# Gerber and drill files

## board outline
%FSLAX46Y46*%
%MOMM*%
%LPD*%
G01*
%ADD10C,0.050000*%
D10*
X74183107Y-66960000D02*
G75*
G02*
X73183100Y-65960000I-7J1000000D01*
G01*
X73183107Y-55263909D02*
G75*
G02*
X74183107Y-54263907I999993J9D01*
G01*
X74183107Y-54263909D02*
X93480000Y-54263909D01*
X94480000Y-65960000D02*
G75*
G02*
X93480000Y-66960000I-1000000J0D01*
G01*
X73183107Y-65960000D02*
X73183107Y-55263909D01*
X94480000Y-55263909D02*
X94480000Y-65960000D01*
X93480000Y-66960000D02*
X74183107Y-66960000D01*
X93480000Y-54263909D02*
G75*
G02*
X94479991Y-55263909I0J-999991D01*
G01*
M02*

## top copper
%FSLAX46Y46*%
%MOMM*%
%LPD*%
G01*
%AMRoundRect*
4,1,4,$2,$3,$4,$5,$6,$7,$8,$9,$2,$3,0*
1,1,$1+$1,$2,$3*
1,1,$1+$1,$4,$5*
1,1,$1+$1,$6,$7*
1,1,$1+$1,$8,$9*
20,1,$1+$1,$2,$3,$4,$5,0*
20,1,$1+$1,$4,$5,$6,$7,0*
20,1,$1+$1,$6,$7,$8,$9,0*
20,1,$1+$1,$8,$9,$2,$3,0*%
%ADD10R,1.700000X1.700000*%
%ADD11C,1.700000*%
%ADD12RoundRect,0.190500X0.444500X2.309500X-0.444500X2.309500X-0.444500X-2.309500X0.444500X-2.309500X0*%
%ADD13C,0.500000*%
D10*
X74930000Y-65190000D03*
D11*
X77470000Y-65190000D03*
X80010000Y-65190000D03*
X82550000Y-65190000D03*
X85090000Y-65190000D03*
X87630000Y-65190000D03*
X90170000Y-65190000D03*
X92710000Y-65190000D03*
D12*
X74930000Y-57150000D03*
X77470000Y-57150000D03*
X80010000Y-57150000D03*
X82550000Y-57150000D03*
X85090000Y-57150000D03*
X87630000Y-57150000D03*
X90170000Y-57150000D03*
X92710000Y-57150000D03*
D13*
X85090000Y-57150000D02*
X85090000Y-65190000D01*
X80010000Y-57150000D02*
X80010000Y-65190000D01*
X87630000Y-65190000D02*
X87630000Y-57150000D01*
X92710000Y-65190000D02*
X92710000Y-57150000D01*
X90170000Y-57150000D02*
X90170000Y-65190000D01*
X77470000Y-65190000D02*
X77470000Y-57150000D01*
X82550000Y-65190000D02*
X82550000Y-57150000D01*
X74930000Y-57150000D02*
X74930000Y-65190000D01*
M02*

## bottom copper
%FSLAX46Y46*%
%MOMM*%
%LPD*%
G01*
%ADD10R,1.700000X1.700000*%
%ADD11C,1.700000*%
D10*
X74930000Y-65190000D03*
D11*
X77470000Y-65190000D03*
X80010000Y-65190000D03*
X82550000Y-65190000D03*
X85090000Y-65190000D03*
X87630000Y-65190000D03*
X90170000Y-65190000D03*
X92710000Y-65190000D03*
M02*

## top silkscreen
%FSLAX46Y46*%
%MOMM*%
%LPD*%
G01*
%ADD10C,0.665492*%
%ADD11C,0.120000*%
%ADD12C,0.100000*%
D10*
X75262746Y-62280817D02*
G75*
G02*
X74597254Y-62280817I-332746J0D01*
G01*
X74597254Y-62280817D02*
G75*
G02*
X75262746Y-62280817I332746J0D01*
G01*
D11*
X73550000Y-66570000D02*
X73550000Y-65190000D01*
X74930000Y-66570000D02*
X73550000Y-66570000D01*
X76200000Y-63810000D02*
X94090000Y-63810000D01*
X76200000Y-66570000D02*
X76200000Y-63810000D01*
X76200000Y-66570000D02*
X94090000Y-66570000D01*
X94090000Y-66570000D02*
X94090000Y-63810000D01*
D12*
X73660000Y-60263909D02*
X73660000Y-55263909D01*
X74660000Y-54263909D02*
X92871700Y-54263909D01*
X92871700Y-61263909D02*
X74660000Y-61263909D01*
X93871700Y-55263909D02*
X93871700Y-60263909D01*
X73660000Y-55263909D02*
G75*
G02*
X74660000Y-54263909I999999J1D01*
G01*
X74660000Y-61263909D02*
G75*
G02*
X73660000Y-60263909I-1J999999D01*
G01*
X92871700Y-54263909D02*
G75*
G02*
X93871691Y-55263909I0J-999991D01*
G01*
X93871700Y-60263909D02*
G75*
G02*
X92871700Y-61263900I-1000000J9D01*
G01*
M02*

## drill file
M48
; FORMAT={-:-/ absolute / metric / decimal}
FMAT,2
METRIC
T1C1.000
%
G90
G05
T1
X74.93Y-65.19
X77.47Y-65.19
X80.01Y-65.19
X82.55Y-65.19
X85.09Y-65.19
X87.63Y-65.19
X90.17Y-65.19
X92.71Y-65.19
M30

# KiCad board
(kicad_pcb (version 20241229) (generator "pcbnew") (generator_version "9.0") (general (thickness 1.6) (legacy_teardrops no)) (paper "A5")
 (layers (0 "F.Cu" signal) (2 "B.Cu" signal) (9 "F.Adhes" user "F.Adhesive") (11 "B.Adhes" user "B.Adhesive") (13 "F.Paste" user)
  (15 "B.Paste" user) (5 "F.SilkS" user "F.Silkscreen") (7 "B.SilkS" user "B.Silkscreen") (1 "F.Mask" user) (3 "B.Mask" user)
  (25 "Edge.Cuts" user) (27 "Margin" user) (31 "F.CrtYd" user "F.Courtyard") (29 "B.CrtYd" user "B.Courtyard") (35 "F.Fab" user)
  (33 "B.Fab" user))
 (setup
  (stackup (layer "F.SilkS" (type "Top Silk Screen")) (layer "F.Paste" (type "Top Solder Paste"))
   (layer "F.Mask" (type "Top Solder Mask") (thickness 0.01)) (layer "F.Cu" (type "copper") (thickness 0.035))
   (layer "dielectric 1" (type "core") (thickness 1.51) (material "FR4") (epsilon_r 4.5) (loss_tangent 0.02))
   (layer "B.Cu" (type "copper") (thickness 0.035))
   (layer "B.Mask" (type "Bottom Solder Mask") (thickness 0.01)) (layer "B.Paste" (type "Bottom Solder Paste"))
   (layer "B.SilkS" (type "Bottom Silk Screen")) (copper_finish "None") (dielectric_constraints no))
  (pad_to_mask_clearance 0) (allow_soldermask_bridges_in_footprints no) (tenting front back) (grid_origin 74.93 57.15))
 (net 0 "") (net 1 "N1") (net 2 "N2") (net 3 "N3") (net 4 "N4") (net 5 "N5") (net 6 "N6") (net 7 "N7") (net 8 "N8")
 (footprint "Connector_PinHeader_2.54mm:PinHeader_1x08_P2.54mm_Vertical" (layer "F.Cu") (at 74.93 65.19 90)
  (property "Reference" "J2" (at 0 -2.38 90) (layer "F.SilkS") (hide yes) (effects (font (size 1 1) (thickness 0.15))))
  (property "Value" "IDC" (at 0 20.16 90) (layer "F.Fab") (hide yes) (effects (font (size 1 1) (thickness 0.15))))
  (fp_line (start -1.38 -1.38) (end 0 -1.38) (stroke (width 0.12) (type solid)) (layer "F.SilkS"))
  (fp_line (start -1.38 0) (end -1.38 -1.38) (stroke (width 0.12) (type solid)) (layer "F.SilkS"))
  (fp_line (start 1.38 1.27) (end 1.38 19.16) (stroke (width 0.12) (type solid)) (layer "F.SilkS"))
  (fp_line (start -1.38 1.27) (end 1.38 1.27) (stroke (width 0.12) (type solid)) (layer "F.SilkS"))
  (fp_line (start -1.38 1.27) (end -1.38 19.16) (stroke (width 0.12) (type solid)) (layer "F.SilkS"))
  (fp_line (start -1.38 19.16) (end 1.38 19.16) (stroke (width 0.12) (type solid)) (layer "F.SilkS"))
  (pad "1" thru_hole rect (at 0 0 90) (size 1.7 1.7) (drill 1) (layers "*.Cu" "*.Mask") (remove_unused_layers no) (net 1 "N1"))
  (pad "2" thru_hole circle (at 0 2.54 90) (size 1.7 1.7) (drill 1) (layers "*.Cu" "*.Mask") (remove_unused_layers no) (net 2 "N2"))
  (pad "3" thru_hole circle (at 0 5.08 90) (size 1.7 1.7) (drill 1) (layers "*.Cu" "*.Mask") (remove_unused_layers no) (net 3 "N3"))
  (pad "4" thru_hole circle (at 0 7.62 90) (size 1.7 1.7) (drill 1) (layers "*.Cu" "*.Mask") (remove_unused_layers no) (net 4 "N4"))
  (pad "5" thru_hole circle (at 0 10.16 90) (size 1.7 1.7) (drill 1) (layers "*.Cu" "*.Mask") (remove_unused_layers no) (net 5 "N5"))
  (pad "6" thru_hole circle (at 0 12.7 90) (size 1.7 1.7) (drill 1) (layers "*.Cu" "*.Mask") (remove_unused_layers no) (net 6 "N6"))
  (pad "7" thru_hole circle (at 0 15.24 90) (size 1.7 1.7) (drill 1) (layers "*.Cu" "*.Mask") (remove_unused_layers no) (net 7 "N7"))
  (pad "8" thru_hole circle (at 0 17.78 90) (size 1.7 1.7) (drill 1) (layers "*.Cu" "*.Mask") (remove_unused_layers no) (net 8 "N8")))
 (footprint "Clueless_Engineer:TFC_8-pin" (layer "F.Cu") (at 83.82 57.15)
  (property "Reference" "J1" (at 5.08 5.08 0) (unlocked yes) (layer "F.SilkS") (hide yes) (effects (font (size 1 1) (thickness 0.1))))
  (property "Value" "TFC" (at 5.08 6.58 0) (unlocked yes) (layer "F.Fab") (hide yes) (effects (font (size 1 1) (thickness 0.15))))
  (fp_line (start -10.16 3.113909) (end -10.16 -1.886091) (stroke (width 0.1) (type default)) (layer "F.SilkS"))
  (fp_line (start -9.16 -2.886091) (end 9.0517 -2.886091) (stroke (width 0.1) (type default)) (layer "F.SilkS"))
  (fp_line (start 9.0517 4.113909) (end -9.16 4.113909) (stroke (width 0.1) (type default)) (layer "F.SilkS"))
  (fp_line (start 10.0517 -1.886091) (end 10.0517 3.113909) (stroke (width 0.1) (type default)) (layer "F.SilkS"))
  (fp_arc (start -10.16 -1.886091) (mid -9.867107 -2.593198) (end -9.16 -2.886091) (stroke (width 0.1) (type default)) (layer "F.SilkS"))
  (fp_arc (start -9.16 4.113909) (mid -9.867107 3.821016) (end -10.16 3.113909) (stroke (width 0.1) (type default)) (layer "F.SilkS"))
  (fp_arc (start 9.0517 -2.886091) (mid 9.758804 -2.593197) (end 10.0517 -1.886091) (stroke (width 0.1) (type default)) (layer "F.SilkS"))
  (fp_arc (start 10.0517 3.113909) (mid 9.758804 3.82101) (end 9.0517 4.113909) (stroke (width 0.1) (type default)) (layer "F.SilkS"))
  (pad "1" connect roundrect (at -8.89 0 180) (size 1.27 5) (layers "F.Cu" "F.Mask") (roundrect_rratio 0.15) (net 1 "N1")
   (thermal_bridge_angle 45))
  (pad "2" connect roundrect (at -6.35 0 180) (size 1.27 5) (layers "F.Cu" "F.Mask") (roundrect_rratio 0.15) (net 2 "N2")
   (thermal_bridge_angle 45))
  (pad "3" connect roundrect (at -3.81 0 180) (size 1.27 5) (layers "F.Cu" "F.Mask") (roundrect_rratio 0.15) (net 3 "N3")
   (thermal_bridge_angle 45))
  (pad "4" connect roundrect (at -1.27 0 180) (size 1.27 5) (layers "F.Cu" "F.Mask") (roundrect_rratio 0.15) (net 4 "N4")
   (thermal_bridge_angle 45))
  (pad "5" connect roundrect (at 1.27 0 180) (size 1.27 5) (layers "F.Cu" "F.Mask") (roundrect_rratio 0.15) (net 5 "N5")
   (thermal_bridge_angle 45))
  (pad "6" connect roundrect (at 3.81 0 180) (size 1.27 5) (layers "F.Cu" "F.Mask") (roundrect_rratio 0.15) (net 6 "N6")
   (thermal_bridge_angle 45))
  (pad "7" connect roundrect (at 6.35 0 180) (size 1.27 5) (layers "F.Cu" "F.Mask") (roundrect_rratio 0.15) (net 7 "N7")
   (thermal_bridge_angle 45))
  (pad "8" connect roundrect (at 8.89 0 180) (size 1.27 5) (layers "F.Cu" "F.Mask") (roundrect_rratio 0.15) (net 8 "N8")
   (thermal_bridge_angle 45)))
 (gr_circle (center 74.93 62.280817) (end 75.530484 62.415908) (stroke (width 0.1) (type solid)) (fill yes) (layer "F.SilkS"))
 (gr_arc (start 74.183107 66.96) (mid 73.475996 66.667109) (end 73.183107 65.96) (stroke (width 0.05) (type default)) (layer "Edge.Cuts"))
 (gr_arc (start 73.183107 55.263909) (mid 73.476 54.556802) (end 74.183107 54.263909) (stroke (width 0.05) (type default))
  (layer "Edge.Cuts"))
 (gr_line (start 74.183107 54.263909) (end 93.48 54.263909) (stroke (width 0.05) (type default)) (layer "Edge.Cuts"))
 (gr_arc (start 94.48 65.96) (mid 94.187107 66.667107) (end 93.48 66.96) (stroke (width 0.05) (type default)) (layer "Edge.Cuts"))
 (gr_line (start 73.183107 65.96) (end 73.183107 55.263909) (stroke (width 0.05) (type default)) (layer "Edge.Cuts"))
 (gr_line (start 94.48 55.263909) (end 94.48 65.96) (stroke (width 0.05) (type default)) (layer "Edge.Cuts"))
 (gr_line (start 93.48 66.96) (end 74.183107 66.96) (stroke (width 0.05) (type default)) (layer "Edge.Cuts"))
 (gr_arc (start 93.48 54.263909) (mid 94.187104 54.556803) (end 94.48 55.263909) (stroke (width 0.05) (type default)) (layer "Edge.Cuts"))
 (segment (start 85.09 57.15) (end 85.09 65.19) (width 0.5) (layer "F.Cu") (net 5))
 (segment (start 80.01 57.15) (end 80.01 65.19) (width 0.5) (layer "F.Cu") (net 3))
 (segment (start 87.63 65.19) (end 87.63 57.15) (width 0.5) (layer "F.Cu") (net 6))
 (segment (start 92.71 65.19) (end 92.71 57.15) (width 0.5) (layer "F.Cu") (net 8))
 (segment (start 90.17 57.15) (end 90.17 65.19) (width 0.5) (layer "F.Cu") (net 7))
 (segment (start 77.47 65.19) (end 77.47 57.15) (width 0.5) (layer "F.Cu") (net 2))
 (segment (start 82.55 65.19) (end 82.55 57.15) (width 0.5) (layer "F.Cu") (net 4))
 (segment (start 74.93 57.15) (end 74.93 65.19) (width 0.5) (layer "F.Cu") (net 1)))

